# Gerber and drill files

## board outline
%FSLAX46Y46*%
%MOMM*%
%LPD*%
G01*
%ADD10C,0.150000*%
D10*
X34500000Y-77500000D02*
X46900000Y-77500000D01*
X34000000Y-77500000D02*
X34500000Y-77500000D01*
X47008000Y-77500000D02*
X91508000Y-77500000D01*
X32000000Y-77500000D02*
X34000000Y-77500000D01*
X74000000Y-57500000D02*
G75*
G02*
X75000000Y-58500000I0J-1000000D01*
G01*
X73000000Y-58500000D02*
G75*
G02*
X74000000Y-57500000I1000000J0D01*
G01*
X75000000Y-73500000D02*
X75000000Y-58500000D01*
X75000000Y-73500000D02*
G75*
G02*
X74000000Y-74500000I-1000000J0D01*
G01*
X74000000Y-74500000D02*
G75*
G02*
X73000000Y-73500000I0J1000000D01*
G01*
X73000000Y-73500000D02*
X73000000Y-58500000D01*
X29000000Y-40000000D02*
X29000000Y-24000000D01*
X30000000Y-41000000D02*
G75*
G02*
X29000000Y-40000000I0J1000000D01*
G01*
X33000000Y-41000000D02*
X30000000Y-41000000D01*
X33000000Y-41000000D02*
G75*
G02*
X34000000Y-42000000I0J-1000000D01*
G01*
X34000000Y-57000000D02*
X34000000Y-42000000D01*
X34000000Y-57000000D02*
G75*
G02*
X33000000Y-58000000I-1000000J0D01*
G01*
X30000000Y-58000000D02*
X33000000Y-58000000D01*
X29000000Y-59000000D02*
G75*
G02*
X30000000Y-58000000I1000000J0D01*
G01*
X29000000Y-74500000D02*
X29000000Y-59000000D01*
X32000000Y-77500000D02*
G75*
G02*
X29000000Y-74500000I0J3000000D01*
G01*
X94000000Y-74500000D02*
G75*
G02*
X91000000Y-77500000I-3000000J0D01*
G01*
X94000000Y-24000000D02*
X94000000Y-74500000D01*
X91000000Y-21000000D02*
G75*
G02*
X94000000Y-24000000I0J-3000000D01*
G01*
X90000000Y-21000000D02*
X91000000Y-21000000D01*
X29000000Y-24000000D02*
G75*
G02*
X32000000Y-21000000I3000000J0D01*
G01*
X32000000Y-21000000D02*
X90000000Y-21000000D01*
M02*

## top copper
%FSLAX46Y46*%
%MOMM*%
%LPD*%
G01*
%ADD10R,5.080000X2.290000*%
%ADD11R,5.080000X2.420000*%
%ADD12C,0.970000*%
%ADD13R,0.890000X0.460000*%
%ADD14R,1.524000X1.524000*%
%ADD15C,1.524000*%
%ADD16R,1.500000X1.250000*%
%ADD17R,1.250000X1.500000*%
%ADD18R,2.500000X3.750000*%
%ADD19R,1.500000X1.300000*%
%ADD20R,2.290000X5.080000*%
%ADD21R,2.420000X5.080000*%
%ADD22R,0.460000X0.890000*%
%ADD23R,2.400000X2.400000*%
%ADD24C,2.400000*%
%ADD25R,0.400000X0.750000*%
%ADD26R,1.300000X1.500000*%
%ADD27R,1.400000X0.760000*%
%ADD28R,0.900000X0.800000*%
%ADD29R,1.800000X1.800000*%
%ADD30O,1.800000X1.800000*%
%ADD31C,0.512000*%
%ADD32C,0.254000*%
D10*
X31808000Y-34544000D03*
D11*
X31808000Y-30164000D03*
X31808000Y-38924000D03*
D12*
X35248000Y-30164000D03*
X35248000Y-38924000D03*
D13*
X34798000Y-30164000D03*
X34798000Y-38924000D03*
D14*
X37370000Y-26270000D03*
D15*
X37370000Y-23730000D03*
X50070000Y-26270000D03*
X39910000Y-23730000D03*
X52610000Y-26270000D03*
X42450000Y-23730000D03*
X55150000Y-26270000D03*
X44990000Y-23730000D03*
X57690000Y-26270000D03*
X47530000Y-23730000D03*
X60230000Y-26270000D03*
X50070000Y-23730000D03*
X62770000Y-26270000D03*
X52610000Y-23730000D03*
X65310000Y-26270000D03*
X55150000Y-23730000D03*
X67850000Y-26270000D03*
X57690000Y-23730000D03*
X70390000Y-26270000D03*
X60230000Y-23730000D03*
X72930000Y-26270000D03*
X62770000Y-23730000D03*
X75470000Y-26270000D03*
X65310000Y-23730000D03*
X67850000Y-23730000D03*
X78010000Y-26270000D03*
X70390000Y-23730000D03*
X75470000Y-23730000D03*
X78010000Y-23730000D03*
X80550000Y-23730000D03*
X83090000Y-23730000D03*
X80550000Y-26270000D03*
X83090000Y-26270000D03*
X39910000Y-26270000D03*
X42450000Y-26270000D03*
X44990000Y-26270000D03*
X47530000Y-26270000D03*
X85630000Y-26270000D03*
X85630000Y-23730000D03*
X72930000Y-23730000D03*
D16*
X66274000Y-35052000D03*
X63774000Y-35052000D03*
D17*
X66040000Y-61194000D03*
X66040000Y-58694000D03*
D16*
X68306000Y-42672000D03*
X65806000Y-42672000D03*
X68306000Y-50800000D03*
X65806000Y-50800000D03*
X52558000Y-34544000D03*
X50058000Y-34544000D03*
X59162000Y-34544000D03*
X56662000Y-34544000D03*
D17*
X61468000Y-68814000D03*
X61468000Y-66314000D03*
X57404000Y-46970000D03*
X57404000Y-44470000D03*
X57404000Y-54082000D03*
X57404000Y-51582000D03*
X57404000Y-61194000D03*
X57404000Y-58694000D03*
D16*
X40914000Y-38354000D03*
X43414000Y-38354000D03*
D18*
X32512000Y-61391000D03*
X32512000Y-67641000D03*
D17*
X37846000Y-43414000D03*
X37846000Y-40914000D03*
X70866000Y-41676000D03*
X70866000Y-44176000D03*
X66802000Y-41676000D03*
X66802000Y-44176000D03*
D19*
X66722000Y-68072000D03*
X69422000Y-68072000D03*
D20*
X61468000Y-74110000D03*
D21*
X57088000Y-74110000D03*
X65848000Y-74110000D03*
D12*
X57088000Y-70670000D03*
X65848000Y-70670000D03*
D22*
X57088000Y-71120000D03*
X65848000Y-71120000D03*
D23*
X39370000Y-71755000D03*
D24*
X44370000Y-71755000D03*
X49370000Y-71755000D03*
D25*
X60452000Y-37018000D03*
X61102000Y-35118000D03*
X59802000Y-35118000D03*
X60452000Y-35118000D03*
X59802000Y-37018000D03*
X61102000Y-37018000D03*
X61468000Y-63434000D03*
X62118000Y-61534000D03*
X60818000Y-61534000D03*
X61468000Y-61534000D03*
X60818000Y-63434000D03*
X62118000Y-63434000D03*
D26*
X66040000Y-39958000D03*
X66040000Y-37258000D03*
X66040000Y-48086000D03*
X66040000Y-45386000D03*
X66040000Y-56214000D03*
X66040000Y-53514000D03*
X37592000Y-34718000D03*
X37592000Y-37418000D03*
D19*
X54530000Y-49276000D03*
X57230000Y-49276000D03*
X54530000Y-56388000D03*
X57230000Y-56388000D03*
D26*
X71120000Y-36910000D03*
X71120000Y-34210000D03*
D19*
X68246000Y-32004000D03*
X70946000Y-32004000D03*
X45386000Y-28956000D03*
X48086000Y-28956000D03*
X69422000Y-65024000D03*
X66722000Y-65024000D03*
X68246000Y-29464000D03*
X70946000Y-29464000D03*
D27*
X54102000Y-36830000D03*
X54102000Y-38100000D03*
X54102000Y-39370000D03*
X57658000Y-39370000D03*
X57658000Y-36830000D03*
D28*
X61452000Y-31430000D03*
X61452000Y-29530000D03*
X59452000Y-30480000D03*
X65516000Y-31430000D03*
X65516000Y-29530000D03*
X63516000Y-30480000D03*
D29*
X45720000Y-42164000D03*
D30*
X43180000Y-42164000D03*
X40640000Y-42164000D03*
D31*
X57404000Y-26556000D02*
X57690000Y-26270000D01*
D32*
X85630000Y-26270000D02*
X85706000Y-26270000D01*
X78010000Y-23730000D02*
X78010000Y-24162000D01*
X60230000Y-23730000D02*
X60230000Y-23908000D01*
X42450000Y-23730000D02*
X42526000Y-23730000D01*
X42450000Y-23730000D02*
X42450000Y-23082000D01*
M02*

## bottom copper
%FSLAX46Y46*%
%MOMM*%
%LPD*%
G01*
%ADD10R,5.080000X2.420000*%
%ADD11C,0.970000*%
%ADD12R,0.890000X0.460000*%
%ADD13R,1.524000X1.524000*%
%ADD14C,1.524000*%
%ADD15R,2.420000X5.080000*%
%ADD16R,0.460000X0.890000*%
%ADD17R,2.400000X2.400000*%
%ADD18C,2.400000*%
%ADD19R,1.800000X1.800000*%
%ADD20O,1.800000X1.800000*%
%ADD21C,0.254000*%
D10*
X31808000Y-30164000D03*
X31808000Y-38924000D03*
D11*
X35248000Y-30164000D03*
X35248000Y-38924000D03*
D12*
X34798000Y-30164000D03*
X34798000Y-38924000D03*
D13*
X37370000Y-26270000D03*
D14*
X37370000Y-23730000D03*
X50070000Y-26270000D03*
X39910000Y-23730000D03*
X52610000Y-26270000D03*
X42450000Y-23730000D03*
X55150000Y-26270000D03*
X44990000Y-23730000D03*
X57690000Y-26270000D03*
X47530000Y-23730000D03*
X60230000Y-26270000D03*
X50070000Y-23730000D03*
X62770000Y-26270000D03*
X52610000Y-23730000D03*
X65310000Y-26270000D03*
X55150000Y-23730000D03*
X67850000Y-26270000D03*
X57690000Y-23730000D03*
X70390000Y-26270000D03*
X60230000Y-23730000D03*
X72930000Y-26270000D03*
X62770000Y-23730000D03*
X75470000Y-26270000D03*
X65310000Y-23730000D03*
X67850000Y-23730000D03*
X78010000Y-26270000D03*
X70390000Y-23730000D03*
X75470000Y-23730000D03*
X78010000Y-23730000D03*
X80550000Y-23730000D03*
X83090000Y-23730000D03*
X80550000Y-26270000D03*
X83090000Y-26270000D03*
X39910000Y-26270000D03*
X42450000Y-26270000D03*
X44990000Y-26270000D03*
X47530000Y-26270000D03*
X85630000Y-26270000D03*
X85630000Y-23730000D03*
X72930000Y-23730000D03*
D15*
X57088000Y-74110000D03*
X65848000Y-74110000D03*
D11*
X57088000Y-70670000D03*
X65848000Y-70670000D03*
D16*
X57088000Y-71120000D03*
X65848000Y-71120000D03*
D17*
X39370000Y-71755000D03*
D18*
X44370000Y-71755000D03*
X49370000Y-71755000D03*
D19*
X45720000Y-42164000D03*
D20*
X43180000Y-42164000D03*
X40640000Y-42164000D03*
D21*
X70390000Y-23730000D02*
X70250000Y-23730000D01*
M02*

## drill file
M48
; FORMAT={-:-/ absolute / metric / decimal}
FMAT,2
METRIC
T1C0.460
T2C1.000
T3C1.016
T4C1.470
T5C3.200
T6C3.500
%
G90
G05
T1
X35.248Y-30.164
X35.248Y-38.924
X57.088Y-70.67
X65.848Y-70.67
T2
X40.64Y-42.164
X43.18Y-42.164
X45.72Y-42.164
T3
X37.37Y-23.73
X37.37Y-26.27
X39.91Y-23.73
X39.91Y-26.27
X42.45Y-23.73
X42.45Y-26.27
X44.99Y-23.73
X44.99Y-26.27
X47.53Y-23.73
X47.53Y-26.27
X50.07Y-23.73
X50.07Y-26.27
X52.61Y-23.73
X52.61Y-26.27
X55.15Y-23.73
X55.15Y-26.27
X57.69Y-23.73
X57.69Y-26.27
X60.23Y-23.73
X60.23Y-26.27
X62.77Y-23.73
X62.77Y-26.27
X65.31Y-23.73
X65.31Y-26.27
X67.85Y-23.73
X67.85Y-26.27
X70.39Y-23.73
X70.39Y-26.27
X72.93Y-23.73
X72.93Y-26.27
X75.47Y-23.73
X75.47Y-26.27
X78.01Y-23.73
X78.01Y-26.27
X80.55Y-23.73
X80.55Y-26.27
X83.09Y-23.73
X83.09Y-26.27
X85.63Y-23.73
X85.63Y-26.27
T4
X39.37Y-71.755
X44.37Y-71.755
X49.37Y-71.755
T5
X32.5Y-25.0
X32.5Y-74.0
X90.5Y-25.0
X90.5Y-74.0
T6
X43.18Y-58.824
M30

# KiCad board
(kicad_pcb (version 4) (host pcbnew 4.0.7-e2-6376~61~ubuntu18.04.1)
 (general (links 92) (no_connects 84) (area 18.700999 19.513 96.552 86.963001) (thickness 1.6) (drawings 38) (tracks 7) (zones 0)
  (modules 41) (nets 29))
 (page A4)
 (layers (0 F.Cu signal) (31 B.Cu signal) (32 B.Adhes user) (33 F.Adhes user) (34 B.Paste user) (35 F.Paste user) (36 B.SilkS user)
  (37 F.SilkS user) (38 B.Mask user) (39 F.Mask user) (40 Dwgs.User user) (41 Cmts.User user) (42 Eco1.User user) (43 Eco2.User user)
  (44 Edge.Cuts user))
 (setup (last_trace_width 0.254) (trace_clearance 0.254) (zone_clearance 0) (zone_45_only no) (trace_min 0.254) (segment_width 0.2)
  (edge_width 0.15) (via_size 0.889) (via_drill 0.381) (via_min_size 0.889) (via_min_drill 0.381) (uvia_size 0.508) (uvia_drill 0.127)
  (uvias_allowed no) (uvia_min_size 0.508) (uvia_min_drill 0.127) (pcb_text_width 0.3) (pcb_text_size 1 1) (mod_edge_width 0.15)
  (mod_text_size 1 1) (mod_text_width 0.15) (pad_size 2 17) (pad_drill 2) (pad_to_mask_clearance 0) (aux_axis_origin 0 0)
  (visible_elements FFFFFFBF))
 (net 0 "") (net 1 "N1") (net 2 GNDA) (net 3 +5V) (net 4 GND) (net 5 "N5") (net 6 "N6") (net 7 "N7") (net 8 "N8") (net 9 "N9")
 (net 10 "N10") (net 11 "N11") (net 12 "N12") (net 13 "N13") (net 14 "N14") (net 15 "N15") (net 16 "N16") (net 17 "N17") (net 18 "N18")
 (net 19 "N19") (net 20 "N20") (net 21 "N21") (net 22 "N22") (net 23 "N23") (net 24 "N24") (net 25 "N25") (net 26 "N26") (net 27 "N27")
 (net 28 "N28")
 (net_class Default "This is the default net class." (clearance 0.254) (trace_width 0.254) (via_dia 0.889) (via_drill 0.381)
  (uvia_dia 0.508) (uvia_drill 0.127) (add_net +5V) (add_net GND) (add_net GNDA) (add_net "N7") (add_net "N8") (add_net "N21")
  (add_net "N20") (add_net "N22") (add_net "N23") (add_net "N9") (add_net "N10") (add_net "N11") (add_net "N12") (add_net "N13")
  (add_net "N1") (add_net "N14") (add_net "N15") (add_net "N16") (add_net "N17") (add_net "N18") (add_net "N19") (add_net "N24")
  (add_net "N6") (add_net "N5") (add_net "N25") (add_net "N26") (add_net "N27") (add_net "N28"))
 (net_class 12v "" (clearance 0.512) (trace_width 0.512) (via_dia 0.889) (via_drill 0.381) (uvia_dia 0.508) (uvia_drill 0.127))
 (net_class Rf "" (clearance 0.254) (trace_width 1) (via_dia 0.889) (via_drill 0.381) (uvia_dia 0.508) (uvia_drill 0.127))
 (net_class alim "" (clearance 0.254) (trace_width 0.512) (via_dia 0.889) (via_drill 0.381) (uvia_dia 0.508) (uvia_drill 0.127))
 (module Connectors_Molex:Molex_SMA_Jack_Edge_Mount (layer F.Cu) (at 33.528 34.544)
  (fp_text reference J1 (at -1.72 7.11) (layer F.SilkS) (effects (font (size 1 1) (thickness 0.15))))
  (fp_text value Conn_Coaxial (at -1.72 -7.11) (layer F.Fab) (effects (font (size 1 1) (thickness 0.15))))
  (pad 1 smd rect (at -1.72 0) (size 5.08 2.29) (layers F.Cu F.Paste F.Mask) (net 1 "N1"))
  (pad 2 smd rect (at -1.72 -4.38) (size 5.08 2.42) (layers F.Cu F.Paste F.Mask) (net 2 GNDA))
  (pad 2 smd rect (at -1.72 4.38) (size 5.08 2.42) (layers F.Cu F.Paste F.Mask) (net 2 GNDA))
  (pad 2 smd rect (at -1.72 -4.38) (size 5.08 2.42) (layers B.Cu B.Paste B.Mask) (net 2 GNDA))
  (pad 2 smd rect (at -1.72 4.38) (size 5.08 2.42) (layers B.Cu B.Paste B.Mask) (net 2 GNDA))
  (pad 2 thru_hole circle (at 1.72 -4.38) (size 0.97 0.97) (drill 0.46) (layers *.Cu) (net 2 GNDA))
  (pad 2 thru_hole circle (at 1.72 4.38) (size 0.97 0.97) (drill 0.46) (layers *.Cu) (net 2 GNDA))
  (pad 2 smd rect (at 1.27 -4.38) (size 0.89 0.46) (layers F.Cu) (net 2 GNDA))
  (pad 2 smd rect (at 1.27 4.38) (size 0.89 0.46) (layers F.Cu) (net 2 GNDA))
  (pad 2 smd rect (at 1.27 -4.38) (size 0.89 0.46) (layers B.Cu) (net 2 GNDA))
  (pad 2 smd rect (at 1.27 4.38) (size 0.89 0.46) (layers B.Cu) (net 2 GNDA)))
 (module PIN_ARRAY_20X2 (layer F.Cu) (at 61.5 25)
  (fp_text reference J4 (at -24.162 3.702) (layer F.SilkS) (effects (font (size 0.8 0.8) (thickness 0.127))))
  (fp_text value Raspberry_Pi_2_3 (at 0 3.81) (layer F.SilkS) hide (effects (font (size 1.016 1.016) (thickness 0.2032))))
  (pad 1 thru_hole rect (at -24.13 1.27) (size 1.524 1.524) (drill 1.016) (layers *.Cu *.Mask F.SilkS))
  (pad 2 thru_hole circle (at -24.13 -1.27) (size 1.524 1.524) (drill 1.016) (layers *.Cu *.Mask F.SilkS) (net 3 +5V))
  (pad 11 thru_hole circle (at -11.43 1.27) (size 1.524 1.524) (drill 1.016) (layers *.Cu *.Mask F.SilkS))
  (pad 4 thru_hole circle (at -21.59 -1.27) (size 1.524 1.524) (drill 1.016) (layers *.Cu *.Mask F.SilkS) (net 3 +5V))
  (pad 13 thru_hole circle (at -8.89 1.27) (size 1.524 1.524) (drill 1.016) (layers *.Cu *.Mask F.SilkS))
  (pad 6 thru_hole circle (at -19.05 -1.27) (size 1.524 1.524) (drill 1.016) (layers *.Cu *.Mask F.SilkS) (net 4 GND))
  (pad 15 thru_hole circle (at -6.35 1.27) (size 1.524 1.524) (drill 1.016) (layers *.Cu *.Mask F.SilkS))
  (pad 8 thru_hole circle (at -16.51 -1.27) (size 1.524 1.524) (drill 1.016) (layers *.Cu *.Mask F.SilkS) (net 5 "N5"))
  (pad 17 thru_hole circle (at -3.81 1.27) (size 1.524 1.524) (drill 1.016) (layers *.Cu *.Mask F.SilkS))
  (pad 10 thru_hole circle (at -13.97 -1.27) (size 1.524 1.524) (drill 1.016) (layers *.Cu *.Mask F.SilkS) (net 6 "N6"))
  (pad 19 thru_hole circle (at -1.27 1.27) (size 1.524 1.524) (drill 1.016) (layers *.Cu *.Mask F.SilkS))
  (pad 12 thru_hole circle (at -11.43 -1.27) (size 1.524 1.524) (drill 1.016) (layers *.Cu *.Mask F.SilkS))
  (pad 21 thru_hole circle (at 1.27 1.27) (size 1.524 1.524) (drill 1.016) (layers *.Cu *.Mask F.SilkS))
  (pad 14 thru_hole circle (at -8.89 -1.27) (size 1.524 1.524) (drill 1.016) (layers *.Cu *.Mask F.SilkS) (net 4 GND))
  (pad 23 thru_hole circle (at 3.81 1.27) (size 1.524 1.524) (drill 1.016) (layers *.Cu *.Mask F.SilkS))
  (pad 16 thru_hole circle (at -6.35 -1.27) (size 1.524 1.524) (drill 1.016) (layers *.Cu *.Mask F.SilkS))
  (pad 25 thru_hole circle (at 6.35 1.27) (size 1.524 1.524) (drill 1.016) (layers *.Cu *.Mask F.SilkS) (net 4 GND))
  (pad 18 thru_hole circle (at -3.81 -1.27) (size 1.524 1.524) (drill 1.016) (layers *.Cu *.Mask F.SilkS))
  (pad 27 thru_hole circle (at 8.89 1.27) (size 1.524 1.524) (drill 1.016) (layers *.Cu *.Mask F.SilkS))
  (pad 20 thru_hole circle (at -1.27 -1.27) (size 1.524 1.524) (drill 1.016) (layers *.Cu *.Mask F.SilkS) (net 4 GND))
  (pad 29 thru_hole circle (at 11.43 1.27) (size 1.524 1.524) (drill 1.016) (layers *.Cu *.Mask F.SilkS))
  (pad 22 thru_hole circle (at 1.27 -1.27) (size 1.524 1.524) (drill 1.016) (layers *.Cu *.Mask F.SilkS))
  (pad 31 thru_hole circle (at 13.97 1.27) (size 1.524 1.524) (drill 1.016) (layers *.Cu *.Mask F.SilkS))
  (pad 24 thru_hole circle (at 3.81 -1.27) (size 1.524 1.524) (drill 1.016) (layers *.Cu *.Mask F.SilkS))
  (pad 26 thru_hole circle (at 6.35 -1.27) (size 1.524 1.524) (drill 1.016) (layers *.Cu *.Mask F.SilkS))
  (pad 33 thru_hole circle (at 16.51 1.27) (size 1.524 1.524) (drill 1.016) (layers *.Cu *.Mask F.SilkS))
  (pad 28 thru_hole circle (at 8.89 -1.27) (size 1.524 1.524) (drill 1.016) (layers *.Cu *.Mask F.SilkS))
  (pad 32 thru_hole circle (at 13.97 -1.27) (size 1.524 1.524) (drill 1.016) (layers *.Cu *.Mask F.SilkS))
  (pad 34 thru_hole circle (at 16.51 -1.27) (size 1.524 1.524) (drill 1.016) (layers *.Cu *.Mask F.SilkS) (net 4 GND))
  (pad 36 thru_hole circle (at 19.05 -1.27) (size 1.524 1.524) (drill 1.016) (layers *.Cu *.Mask F.SilkS))
  (pad 38 thru_hole circle (at 21.59 -1.27) (size 1.524 1.524) (drill 1.016) (layers *.Cu *.Mask F.SilkS))
  (pad 35 thru_hole circle (at 19.05 1.27) (size 1.524 1.524) (drill 1.016) (layers *.Cu *.Mask F.SilkS))
  (pad 37 thru_hole circle (at 21.59 1.27) (size 1.524 1.524) (drill 1.016) (layers *.Cu *.Mask F.SilkS))
  (pad 3 thru_hole circle (at -21.59 1.27) (size 1.524 1.524) (drill 1.016) (layers *.Cu *.Mask F.SilkS))
  (pad 5 thru_hole circle (at -19.05 1.27) (size 1.524 1.524) (drill 1.016) (layers *.Cu *.Mask F.SilkS))
  (pad 7 thru_hole circle (at -16.51 1.27) (size 1.524 1.524) (drill 1.016) (layers *.Cu *.Mask F.SilkS))
  (pad 9 thru_hole circle (at -13.97 1.27) (size 1.524 1.524) (drill 1.016) (layers *.Cu *.Mask F.SilkS) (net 4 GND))
  (pad 39 thru_hole circle (at 24.13 1.27) (size 1.524 1.524) (drill 1.016) (layers *.Cu *.Mask F.SilkS) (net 4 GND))
  (pad 40 thru_hole circle (at 24.13 -1.27) (size 1.524 1.524) (drill 1.016) (layers *.Cu *.Mask F.SilkS))
  (pad 30 thru_hole circle (at 11.43 -1.27) (size 1.524 1.524) (drill 1.016) (layers *.Cu *.Mask F.SilkS) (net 4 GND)))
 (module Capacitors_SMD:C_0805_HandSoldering (layer F.Cu) (at 65.024 35.052 180)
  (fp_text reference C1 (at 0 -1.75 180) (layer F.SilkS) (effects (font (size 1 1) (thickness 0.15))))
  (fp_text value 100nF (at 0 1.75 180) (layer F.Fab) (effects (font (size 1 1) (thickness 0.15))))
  (pad 1 smd rect (at -1.25 0 180) (size 1.5 1.25) (layers F.Cu F.Paste F.Mask) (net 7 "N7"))
  (pad 2 smd rect (at 1.25 0 180) (size 1.5 1.25) (layers F.Cu F.Paste F.Mask) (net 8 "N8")))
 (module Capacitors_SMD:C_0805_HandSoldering (layer F.Cu) (at 66.04 59.944 90)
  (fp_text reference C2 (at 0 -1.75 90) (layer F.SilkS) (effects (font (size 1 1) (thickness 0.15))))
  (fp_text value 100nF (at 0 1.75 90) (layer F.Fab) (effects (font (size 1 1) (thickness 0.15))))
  (pad 1 smd rect (at -1.25 0 90) (size 1.5 1.25) (layers F.Cu F.Paste F.Mask) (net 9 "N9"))
  (pad 2 smd rect (at 1.25 0 90) (size 1.5 1.25) (layers F.Cu F.Paste F.Mask) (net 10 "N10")))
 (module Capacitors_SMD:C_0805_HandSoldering (layer F.Cu) (at 67.056 42.672 180)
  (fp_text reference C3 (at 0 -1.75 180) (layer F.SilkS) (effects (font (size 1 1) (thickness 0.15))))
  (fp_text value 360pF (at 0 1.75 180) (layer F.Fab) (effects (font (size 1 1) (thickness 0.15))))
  (pad 1 smd rect (at -1.25 0 180) (size 1.5 1.25) (layers F.Cu F.Paste F.Mask) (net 4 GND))
  (pad 2 smd rect (at 1.25 0 180) (size 1.5 1.25) (layers F.Cu F.Paste F.Mask) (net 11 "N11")))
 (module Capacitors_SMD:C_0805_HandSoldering (layer F.Cu) (at 67.056 50.8 180)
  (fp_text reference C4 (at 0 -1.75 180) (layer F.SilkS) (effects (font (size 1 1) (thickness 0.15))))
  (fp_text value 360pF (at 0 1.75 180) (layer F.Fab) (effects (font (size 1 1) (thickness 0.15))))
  (pad 1 smd rect (at -1.25 0 180) (size 1.5 1.25) (layers F.Cu F.Paste F.Mask) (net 4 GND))
  (pad 2 smd rect (at 1.25 0 180) (size 1.5 1.25) (layers F.Cu F.Paste F.Mask) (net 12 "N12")))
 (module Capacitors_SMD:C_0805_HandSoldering (layer F.Cu) (at 51.308 34.544 180)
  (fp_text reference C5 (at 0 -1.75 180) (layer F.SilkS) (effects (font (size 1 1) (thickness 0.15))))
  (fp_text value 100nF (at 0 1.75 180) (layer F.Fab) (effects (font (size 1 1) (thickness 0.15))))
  (pad 1 smd rect (at -1.25 0 180) (size 1.5 1.25) (layers F.Cu F.Paste F.Mask) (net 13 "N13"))
  (pad 2 smd rect (at 1.25 0 180) (size 1.5 1.25) (layers F.Cu F.Paste F.Mask) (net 1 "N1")))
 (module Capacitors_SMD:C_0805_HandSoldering (layer F.Cu) (at 57.912 34.544 180)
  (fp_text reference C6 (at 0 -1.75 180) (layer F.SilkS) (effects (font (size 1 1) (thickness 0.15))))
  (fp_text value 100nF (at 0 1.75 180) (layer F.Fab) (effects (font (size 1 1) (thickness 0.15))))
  (pad 1 smd rect (at -1.25 0 180) (size 1.5 1.25) (layers F.Cu F.Paste F.Mask) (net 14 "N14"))
  (pad 2 smd rect (at 1.25 0 180) (size 1.5 1.25) (layers F.Cu F.Paste F.Mask) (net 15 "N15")))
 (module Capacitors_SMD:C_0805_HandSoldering (layer F.Cu) (at 61.468 67.564 90)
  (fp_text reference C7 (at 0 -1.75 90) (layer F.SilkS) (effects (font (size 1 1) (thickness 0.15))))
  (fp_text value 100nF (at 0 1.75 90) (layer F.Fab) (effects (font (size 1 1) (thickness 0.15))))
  (pad 1 smd rect (at -1.25 0 90) (size 1.5 1.25) (layers F.Cu F.Paste F.Mask) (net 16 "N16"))
  (pad 2 smd rect (at 1.25 0 90) (size 1.5 1.25) (layers F.Cu F.Paste F.Mask) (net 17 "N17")))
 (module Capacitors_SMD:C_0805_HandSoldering (layer F.Cu) (at 57.404 45.72 90)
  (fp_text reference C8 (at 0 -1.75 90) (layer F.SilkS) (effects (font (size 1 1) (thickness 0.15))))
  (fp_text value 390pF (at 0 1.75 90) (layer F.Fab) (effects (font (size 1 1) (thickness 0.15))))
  (pad 1 smd rect (at -1.25 0 90) (size 1.5 1.25) (layers F.Cu F.Paste F.Mask) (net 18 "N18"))
  (pad 2 smd rect (at 1.25 0 90) (size 1.5 1.25) (layers F.Cu F.Paste F.Mask) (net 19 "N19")))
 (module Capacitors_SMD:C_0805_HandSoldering (layer F.Cu) (at 57.404 52.832 90)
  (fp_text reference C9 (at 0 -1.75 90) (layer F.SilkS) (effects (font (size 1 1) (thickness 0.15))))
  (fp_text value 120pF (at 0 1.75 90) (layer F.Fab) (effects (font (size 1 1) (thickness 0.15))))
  (pad 1 smd rect (at -1.25 0 90) (size 1.5 1.25) (layers F.Cu F.Paste F.Mask) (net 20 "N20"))
  (pad 2 smd rect (at 1.25 0 90) (size 1.5 1.25) (layers F.Cu F.Paste F.Mask) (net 18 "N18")))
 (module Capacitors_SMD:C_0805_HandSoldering (layer F.Cu) (at 57.404 59.944 90)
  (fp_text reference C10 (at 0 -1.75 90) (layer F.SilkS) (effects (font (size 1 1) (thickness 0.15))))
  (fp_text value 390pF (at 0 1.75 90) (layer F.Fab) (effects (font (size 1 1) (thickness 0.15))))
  (pad 1 smd rect (at -1.25 0 90) (size 1.5 1.25) (layers F.Cu F.Paste F.Mask) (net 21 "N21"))
  (pad 2 smd rect (at 1.25 0 90) (size 1.5 1.25) (layers F.Cu F.Paste F.Mask) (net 20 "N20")))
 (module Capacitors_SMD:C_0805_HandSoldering (layer F.Cu) (at 42.164 38.354)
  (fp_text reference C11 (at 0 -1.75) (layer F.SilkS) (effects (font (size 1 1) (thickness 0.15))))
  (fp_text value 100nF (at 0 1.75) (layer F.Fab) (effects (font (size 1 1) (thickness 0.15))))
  (pad 1 smd rect (at -1.25 0) (size 1.5 1.25) (layers F.Cu F.Paste F.Mask) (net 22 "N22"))
  (pad 2 smd rect (at 1.25 0) (size 1.5 1.25) (layers F.Cu F.Paste F.Mask) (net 2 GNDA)))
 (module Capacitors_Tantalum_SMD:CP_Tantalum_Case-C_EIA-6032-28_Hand (layer F.Cu) (at 32.512 64.516 270)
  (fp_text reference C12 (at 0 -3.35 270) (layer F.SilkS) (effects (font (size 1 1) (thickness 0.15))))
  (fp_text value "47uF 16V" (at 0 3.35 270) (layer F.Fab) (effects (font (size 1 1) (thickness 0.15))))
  (pad 1 smd rect (at -3.125 0 270) (size 3.75 2.5) (layers F.Cu F.Paste F.Mask) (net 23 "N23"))
  (pad 2 smd rect (at 3.125 0 270) (size 3.75 2.5) (layers F.Cu F.Paste F.Mask) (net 2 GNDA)))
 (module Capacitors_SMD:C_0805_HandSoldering (layer F.Cu) (at 37.846 42.164 90)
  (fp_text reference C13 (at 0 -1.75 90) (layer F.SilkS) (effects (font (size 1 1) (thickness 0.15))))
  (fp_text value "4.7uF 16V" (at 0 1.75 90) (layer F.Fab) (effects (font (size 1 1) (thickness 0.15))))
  (pad 1 smd rect (at -1.25 0 90) (size 1.5 1.25) (layers F.Cu F.Paste F.Mask) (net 22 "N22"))
  (pad 2 smd rect (at 1.25 0 90) (size 1.5 1.25) (layers F.Cu F.Paste F.Mask) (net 2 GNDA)))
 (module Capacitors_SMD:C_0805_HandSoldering (layer F.Cu) (at 70.866 42.926 270)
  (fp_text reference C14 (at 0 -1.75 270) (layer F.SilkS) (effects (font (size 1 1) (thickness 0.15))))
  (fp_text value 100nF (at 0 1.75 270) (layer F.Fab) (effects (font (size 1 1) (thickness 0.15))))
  (pad 1 smd rect (at -1.25 0 270) (size 1.5 1.25) (layers F.Cu F.Paste F.Mask) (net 3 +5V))
  (pad 2 smd rect (at 1.25 0 270) (size 1.5 1.25) (layers F.Cu F.Paste F.Mask) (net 4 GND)))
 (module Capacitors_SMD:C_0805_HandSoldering (layer F.Cu) (at 66.802 42.926 270)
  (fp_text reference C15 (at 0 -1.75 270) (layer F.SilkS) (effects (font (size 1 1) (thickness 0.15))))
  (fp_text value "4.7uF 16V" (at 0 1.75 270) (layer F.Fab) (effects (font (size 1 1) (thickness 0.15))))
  (pad 1 smd rect (at -1.25 0 270) (size 1.5 1.25) (layers F.Cu F.Paste F.Mask) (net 3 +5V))
  (pad 2 smd rect (at 1.25 0 270) (size 1.5 1.25) (layers F.Cu F.Paste F.Mask) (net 4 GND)))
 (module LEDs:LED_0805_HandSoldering (layer F.Cu) (at 68.072 68.072)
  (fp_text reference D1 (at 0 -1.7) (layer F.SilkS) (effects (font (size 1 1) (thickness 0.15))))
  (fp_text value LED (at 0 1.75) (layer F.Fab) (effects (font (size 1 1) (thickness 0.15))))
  (pad 1 smd rect (at -1.35 0) (size 1.5 1.3) (layers F.Cu F.Paste F.Mask) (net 4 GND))
  (pad 2 smd rect (at 1.35 0) (size 1.5 1.3) (layers F.Cu F.Paste F.Mask) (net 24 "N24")))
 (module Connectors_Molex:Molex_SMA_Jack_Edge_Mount (layer F.Cu) (at 61.468 72.39 90)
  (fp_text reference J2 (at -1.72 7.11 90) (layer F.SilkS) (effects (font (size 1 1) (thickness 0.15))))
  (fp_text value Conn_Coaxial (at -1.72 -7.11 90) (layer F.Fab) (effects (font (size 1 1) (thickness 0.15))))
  (pad 1 smd rect (at -1.72 0 90) (size 5.08 2.29) (layers F.Cu F.Paste F.Mask) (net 16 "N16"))
  (pad 2 smd rect (at -1.72 -4.38 90) (size 5.08 2.42) (layers F.Cu F.Paste F.Mask) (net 4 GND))
  (pad 2 smd rect (at -1.72 4.38 90) (size 5.08 2.42) (layers F.Cu F.Paste F.Mask) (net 4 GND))
  (pad 2 smd rect (at -1.72 -4.38 90) (size 5.08 2.42) (layers B.Cu B.Paste B.Mask) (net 4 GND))
  (pad 2 smd rect (at -1.72 4.38 90) (size 5.08 2.42) (layers B.Cu B.Paste B.Mask) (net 4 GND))
  (pad 2 thru_hole circle (at 1.72 -4.38 90) (size 0.97 0.97) (drill 0.46) (layers *.Cu) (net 4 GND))
  (pad 2 thru_hole circle (at 1.72 4.38 90) (size 0.97 0.97) (drill 0.46) (layers *.Cu) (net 4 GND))
  (pad 2 smd rect (at 1.27 -4.38 90) (size 0.89 0.46) (layers F.Cu) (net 4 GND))
  (pad 2 smd rect (at 1.27 4.38 90) (size 0.89 0.46) (layers F.Cu) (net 4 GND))
  (pad 2 smd rect (at 1.27 -4.38 90) (size 0.89 0.46) (layers B.Cu) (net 4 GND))
  (pad 2 smd rect (at 1.27 4.38 90) (size 0.89 0.46) (layers B.Cu) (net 4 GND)))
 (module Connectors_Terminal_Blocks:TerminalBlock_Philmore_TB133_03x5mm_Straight (layer F.Cu) (at 39.37 71.755)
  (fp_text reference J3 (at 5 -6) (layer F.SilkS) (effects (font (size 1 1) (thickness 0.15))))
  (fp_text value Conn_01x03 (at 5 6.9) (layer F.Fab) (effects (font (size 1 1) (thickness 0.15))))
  (pad 1 thru_hole rect (at 0 0) (size 2.4 2.4) (drill 1.47) (layers *.Cu *.Mask) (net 2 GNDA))
  (pad 2 thru_hole circle (at 5 0) (size 2.4 2.4) (drill 1.47) (layers *.Cu *.Mask) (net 23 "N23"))
  (pad 3 thru_hole circle (at 10 0) (size 2.4 2.4) (drill 1.47) (layers *.Cu *.Mask) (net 22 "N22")))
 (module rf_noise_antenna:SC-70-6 (layer F.Cu) (at 60.452 36.068 270)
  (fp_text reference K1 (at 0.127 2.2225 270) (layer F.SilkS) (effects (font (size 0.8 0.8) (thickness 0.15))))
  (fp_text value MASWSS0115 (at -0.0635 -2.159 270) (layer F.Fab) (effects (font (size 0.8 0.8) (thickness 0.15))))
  (pad 5 smd rect (at 0.95 0 90) (size 0.75 0.4) (layers F.Cu F.Paste F.Mask) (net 14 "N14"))
  (pad 1 smd rect (at -0.95 -0.65 90) (size 0.75 0.4) (layers F.Cu F.Paste F.Mask) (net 8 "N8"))
  (pad 3 smd rect (at -0.95 0.65 90) (size 0.75 0.4) (layers F.Cu F.Paste F.Mask) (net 19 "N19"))
  (pad 2 smd rect (at -0.95 0 90) (size 0.75 0.4) (layers F.Cu F.Paste F.Mask) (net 4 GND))
  (pad 4 smd rect (at 0.95 0.65 90) (size 0.75 0.4) (layers F.Cu F.Paste F.Mask) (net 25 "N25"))
  (pad 6 smd rect (at 0.95 -0.65 90) (size 0.75 0.4) (layers F.Cu F.Paste F.Mask) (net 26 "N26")))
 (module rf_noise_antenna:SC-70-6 (layer F.Cu) (at 61.468 62.484 270)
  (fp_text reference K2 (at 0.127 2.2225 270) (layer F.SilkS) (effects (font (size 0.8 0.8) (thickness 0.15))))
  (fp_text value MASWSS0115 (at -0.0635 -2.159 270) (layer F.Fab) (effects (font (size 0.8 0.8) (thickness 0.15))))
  (pad 5 smd rect (at 0.95 0 90) (size 0.75 0.4) (layers F.Cu F.Paste F.Mask) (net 17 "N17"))
  (pad 1 smd rect (at -0.95 -0.65 90) (size 0.75 0.4) (layers F.Cu F.Paste F.Mask) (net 9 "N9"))
  (pad 3 smd rect (at -0.95 0.65 90) (size 0.75 0.4) (layers F.Cu F.Paste F.Mask) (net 21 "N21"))
  (pad 2 smd rect (at -0.95 0 90) (size 0.75 0.4) (layers F.Cu F.Paste F.Mask) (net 4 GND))
  (pad 4 smd rect (at 0.95 0.65 90) (size 0.75 0.4) (layers F.Cu F.Paste F.Mask) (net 25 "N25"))
  (pad 6 smd rect (at 0.95 -0.65 90) (size 0.75 0.4) (layers F.Cu F.Paste F.Mask) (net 26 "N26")))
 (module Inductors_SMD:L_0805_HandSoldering (layer F.Cu) (at 66.04 38.608 90)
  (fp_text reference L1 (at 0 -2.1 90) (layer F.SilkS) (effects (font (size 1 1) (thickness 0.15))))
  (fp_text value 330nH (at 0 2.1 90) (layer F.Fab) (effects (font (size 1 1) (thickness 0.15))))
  (pad 1 smd rect (at -1.35 0 90) (size 1.5 1.3) (layers F.Cu F.Paste F.Mask) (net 11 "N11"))
  (pad 2 smd rect (at 1.35 0 90) (size 1.5 1.3) (layers F.Cu F.Paste F.Mask) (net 7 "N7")))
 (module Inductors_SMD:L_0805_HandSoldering (layer F.Cu) (at 66.04 46.736 90)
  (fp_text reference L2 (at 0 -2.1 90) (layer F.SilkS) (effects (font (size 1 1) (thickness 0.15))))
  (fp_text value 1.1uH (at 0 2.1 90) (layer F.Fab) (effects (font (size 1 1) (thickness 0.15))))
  (pad 1 smd rect (at -1.35 0 90) (size 1.5 1.3) (layers F.Cu F.Paste F.Mask) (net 12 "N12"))
  (pad 2 smd rect (at 1.35 0 90) (size 1.5 1.3) (layers F.Cu F.Paste F.Mask) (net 11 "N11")))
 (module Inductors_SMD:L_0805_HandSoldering (layer F.Cu) (at 66.04 54.864 90)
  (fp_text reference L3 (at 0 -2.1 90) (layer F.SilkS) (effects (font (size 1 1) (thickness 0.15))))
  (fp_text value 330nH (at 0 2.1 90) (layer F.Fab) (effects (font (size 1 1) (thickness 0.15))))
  (pad 1 smd rect (at -1.35 0 90) (size 1.5 1.3) (layers F.Cu F.Paste F.Mask) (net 10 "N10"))
  (pad 2 smd rect (at 1.35 0 90) (size 1.5 1.3) (layers F.Cu F.Paste F.Mask) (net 12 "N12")))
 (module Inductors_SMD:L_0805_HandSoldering (layer F.Cu) (at 37.592 36.068 270)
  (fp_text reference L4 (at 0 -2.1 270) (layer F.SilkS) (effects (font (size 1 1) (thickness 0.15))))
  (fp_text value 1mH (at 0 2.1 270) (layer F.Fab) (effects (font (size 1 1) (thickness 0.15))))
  (pad 1 smd rect (at -1.35 0 270) (size 1.5 1.3) (layers F.Cu F.Paste F.Mask) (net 1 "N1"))
  (pad 2 smd rect (at 1.35 0 270) (size 1.5 1.3) (layers F.Cu F.Paste F.Mask) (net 22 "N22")))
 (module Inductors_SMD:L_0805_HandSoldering (layer F.Cu) (at 55.88 49.276)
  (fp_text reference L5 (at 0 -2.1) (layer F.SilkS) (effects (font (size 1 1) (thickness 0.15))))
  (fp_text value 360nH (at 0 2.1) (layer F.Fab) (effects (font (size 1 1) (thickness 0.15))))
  (pad 1 smd rect (at -1.35 0) (size 1.5 1.3) (layers F.Cu F.Paste F.Mask) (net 4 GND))
  (pad 2 smd rect (at 1.35 0) (size 1.5 1.3) (layers F.Cu F.Paste F.Mask) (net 18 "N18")))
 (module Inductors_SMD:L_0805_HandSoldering (layer F.Cu) (at 55.88 56.388)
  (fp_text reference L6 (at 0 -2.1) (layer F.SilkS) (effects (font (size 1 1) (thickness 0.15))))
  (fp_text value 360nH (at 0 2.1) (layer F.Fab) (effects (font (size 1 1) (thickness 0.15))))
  (pad 1 smd rect (at -1.35 0) (size 1.5 1.3) (layers F.Cu F.Paste F.Mask) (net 4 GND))
  (pad 2 smd rect (at 1.35 0) (size 1.5 1.3) (layers F.Cu F.Paste F.Mask) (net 20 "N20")))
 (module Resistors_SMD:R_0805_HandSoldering (layer F.Cu) (at 71.12 35.56 90)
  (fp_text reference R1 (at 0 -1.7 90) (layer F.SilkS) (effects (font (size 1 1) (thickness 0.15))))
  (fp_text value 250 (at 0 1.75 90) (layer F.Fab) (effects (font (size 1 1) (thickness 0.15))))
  (pad 1 smd rect (at -1.35 0 90) (size 1.5 1.3) (layers F.Cu F.Paste F.Mask) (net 25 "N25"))
  (pad 2 smd rect (at 1.35 0 90) (size 1.5 1.3) (layers F.Cu F.Paste F.Mask) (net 3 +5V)))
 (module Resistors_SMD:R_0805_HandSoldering (layer F.Cu) (at 69.596 32.004)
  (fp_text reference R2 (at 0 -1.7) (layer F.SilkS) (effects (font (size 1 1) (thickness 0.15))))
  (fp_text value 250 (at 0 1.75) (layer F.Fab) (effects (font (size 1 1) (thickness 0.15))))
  (pad 1 smd rect (at -1.35 0) (size 1.5 1.3) (layers F.Cu F.Paste F.Mask) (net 26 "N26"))
  (pad 2 smd rect (at 1.35 0) (size 1.5 1.3) (layers F.Cu F.Paste F.Mask) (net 3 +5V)))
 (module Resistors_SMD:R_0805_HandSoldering (layer F.Cu) (at 46.736 28.956)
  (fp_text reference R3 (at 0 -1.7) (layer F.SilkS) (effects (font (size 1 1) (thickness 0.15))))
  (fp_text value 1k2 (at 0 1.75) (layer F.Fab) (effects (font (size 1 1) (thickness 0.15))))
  (pad 1 smd rect (at -1.35 0) (size 1.5 1.3) (layers F.Cu F.Paste F.Mask) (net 5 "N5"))
  (pad 2 smd rect (at 1.35 0) (size 1.5 1.3) (layers F.Cu F.Paste F.Mask) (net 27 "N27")))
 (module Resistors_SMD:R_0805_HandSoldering (layer F.Cu) (at 68.072 65.024 180)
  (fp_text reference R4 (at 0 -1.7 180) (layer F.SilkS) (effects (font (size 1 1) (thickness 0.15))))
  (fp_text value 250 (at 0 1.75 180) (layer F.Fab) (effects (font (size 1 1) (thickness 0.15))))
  (pad 1 smd rect (at -1.35 0 180) (size 1.5 1.3) (layers F.Cu F.Paste F.Mask) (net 24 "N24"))
  (pad 2 smd rect (at 1.35 0 180) (size 1.5 1.3) (layers F.Cu F.Paste F.Mask) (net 26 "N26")))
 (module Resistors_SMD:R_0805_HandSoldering (layer F.Cu) (at 69.596 29.464)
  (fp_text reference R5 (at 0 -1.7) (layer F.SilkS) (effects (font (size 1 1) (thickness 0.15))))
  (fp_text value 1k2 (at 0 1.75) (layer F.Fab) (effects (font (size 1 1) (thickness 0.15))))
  (pad 1 smd rect (at -1.35 0) (size 1.5 1.3) (layers F.Cu F.Paste F.Mask) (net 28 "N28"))
  (pad 2 smd rect (at 1.35 0) (size 1.5 1.3) (layers F.Cu F.Paste F.Mask) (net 6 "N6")))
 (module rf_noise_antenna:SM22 (layer F.Cu) (at 55.88 38.1)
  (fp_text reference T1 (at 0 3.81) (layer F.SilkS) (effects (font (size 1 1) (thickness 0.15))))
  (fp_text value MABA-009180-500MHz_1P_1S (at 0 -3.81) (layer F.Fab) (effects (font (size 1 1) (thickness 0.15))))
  (pad 1 smd rect (at -1.778 -1.27) (size 1.4 0.76) (layers F.Cu F.Paste F.Mask) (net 13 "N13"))
  (pad 2 smd rect (at -1.778 0) (size 1.4 0.76) (layers F.Cu F.Paste F.Mask))
  (pad 3 smd rect (at -1.778 1.27) (size 1.4 0.76) (layers F.Cu F.Paste F.Mask) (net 2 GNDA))
  (pad 4 smd rect (at 1.778 1.27) (size 1.4 0.76) (layers F.Cu F.Paste F.Mask) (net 4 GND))
  (pad 5 smd rect (at 1.778 -1.27) (size 1.4 0.76) (layers F.Cu F.Paste F.Mask) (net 15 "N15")))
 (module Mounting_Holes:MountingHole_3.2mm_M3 (layer F.Cu) (at 32.5 74)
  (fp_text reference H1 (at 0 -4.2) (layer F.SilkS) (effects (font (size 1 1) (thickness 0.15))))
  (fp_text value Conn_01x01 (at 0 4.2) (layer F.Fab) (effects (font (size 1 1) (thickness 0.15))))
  (pad 1 np_thru_hole circle (at 0 0) (size 3.2 3.2) (drill 3.2) (layers *.Cu *.Mask) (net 4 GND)))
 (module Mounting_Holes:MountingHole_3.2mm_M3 (layer F.Cu) (at 90.5 74)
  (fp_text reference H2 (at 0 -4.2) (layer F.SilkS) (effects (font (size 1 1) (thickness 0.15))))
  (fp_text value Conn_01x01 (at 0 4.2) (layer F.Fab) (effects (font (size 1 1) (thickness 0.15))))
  (pad 1 np_thru_hole circle (at 0 0) (size 3.2 3.2) (drill 3.2) (layers *.Cu *.Mask) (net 4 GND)))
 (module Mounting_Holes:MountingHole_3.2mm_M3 (layer F.Cu) (at 32.5 25)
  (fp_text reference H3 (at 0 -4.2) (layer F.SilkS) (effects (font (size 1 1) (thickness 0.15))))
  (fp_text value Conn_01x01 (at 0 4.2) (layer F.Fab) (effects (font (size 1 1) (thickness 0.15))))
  (pad 1 np_thru_hole circle (at 0 0) (size 3.2 3.2) (drill 3.2) (layers *.Cu *.Mask) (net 4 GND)))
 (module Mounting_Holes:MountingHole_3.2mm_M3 (layer F.Cu) (at 90.5 25)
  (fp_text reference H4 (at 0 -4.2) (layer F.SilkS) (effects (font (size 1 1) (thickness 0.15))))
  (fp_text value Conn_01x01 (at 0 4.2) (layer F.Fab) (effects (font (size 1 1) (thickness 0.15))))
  (pad 1 np_thru_hole circle (at 0 0) (size 3.2 3.2) (drill 3.2) (layers *.Cu *.Mask) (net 4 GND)))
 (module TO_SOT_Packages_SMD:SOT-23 (layer F.Cu) (at 60.452 30.48 180)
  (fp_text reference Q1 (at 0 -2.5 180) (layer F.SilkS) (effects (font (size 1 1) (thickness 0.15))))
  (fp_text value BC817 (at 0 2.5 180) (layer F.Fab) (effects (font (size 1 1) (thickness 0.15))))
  (pad 1 smd rect (at -1 -0.95 180) (size 0.9 0.8) (layers F.Cu F.Paste F.Mask) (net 4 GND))
  (pad 2 smd rect (at -1 0.95 180) (size 0.9 0.8) (layers F.Cu F.Paste F.Mask) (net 27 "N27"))
  (pad 3 smd rect (at 1 0 180) (size 0.9 0.8) (layers F.Cu F.Paste F.Mask) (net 25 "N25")))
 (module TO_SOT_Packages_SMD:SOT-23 (layer F.Cu) (at 64.516 30.48 180)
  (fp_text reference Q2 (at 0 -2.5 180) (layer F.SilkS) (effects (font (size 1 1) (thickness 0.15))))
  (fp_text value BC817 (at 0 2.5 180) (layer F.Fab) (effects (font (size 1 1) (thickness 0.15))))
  (pad 1 smd rect (at -1 -0.95 180) (size 0.9 0.8) (layers F.Cu F.Paste F.Mask) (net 4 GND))
  (pad 2 smd rect (at -1 0.95 180) (size 0.9 0.8) (layers F.Cu F.Paste F.Mask) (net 28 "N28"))
  (pad 3 smd rect (at 1 0 180) (size 0.9 0.8) (layers F.Cu F.Paste F.Mask) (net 26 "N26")))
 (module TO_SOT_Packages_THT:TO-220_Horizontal (layer F.Cu) (at 45.72 42.164 180)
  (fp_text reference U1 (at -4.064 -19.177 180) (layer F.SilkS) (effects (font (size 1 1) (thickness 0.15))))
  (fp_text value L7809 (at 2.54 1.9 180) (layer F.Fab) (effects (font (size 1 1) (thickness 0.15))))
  (pad 0 np_thru_hole oval (at 2.54 -16.66 180) (size 3.5 3.5) (drill 3.5) (layers *.Cu *.Mask))
  (pad 1 thru_hole rect (at 0 0 180) (size 1.8 1.8) (drill 1) (layers *.Cu *.Mask) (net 23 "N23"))
  (pad 2 thru_hole oval (at 2.54 0 180) (size 1.8 1.8) (drill 1) (layers *.Cu *.Mask) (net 2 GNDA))
  (pad 3 thru_hole oval (at 5.08 0 180) (size 1.8 1.8) (drill 1) (layers *.Cu *.Mask) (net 22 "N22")))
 (gr_line (start 34.5 77.5) (end 46.9 77.5) (angle 90) (layer Edge.Cuts) (width 0.15))
 (gr_line (start 34 77.5) (end 34.5 77.5) (angle 90) (layer Edge.Cuts) (width 0.15))
 (gr_line (start 47.008 77.5) (end 91.508 77.5) (angle 90) (layer Edge.Cuts) (width 0.15))
 (gr_line (start 32 77.5) (end 34 77.5) (angle 90) (layer Edge.Cuts) (width 0.15))
 (gr_arc (start 74 58.5) (end 74 57.5) (angle 90) (layer Edge.Cuts) (width 0.15))
 (gr_arc (start 74 58.5) (end 73 58.5) (angle 90) (layer Edge.Cuts) (width 0.15))
 (gr_line (start 75 73.5) (end 75 58.5) (angle 90) (layer Edge.Cuts) (width 0.15))
 (gr_arc (start 74 73.5) (end 75 73.5) (angle 90) (layer Edge.Cuts) (width 0.15))
 (gr_arc (start 74 73.5) (end 74 74.5) (angle 90) (layer Edge.Cuts) (width 0.15))
 (gr_line (start 73 73.5) (end 73 58.5) (angle 90) (layer Edge.Cuts) (width 0.15))
 (gr_line (start 29 40) (end 29 24) (angle 90) (layer Edge.Cuts) (width 0.15))
 (gr_arc (start 30 40) (end 30 41) (angle 90) (layer Edge.Cuts) (width 0.15))
 (gr_line (start 33 41) (end 30 41) (angle 90) (layer Edge.Cuts) (width 0.15))
 (gr_arc (start 33 42) (end 33 41) (angle 90) (layer Edge.Cuts) (width 0.15))
 (gr_line (start 34 57) (end 34 42) (angle 90) (layer Edge.Cuts) (width 0.15))
 (gr_arc (start 33 57) (end 34 57) (angle 90) (layer Edge.Cuts) (width 0.15))
 (gr_line (start 30 58) (end 33 58) (angle 90) (layer Edge.Cuts) (width 0.15))
 (gr_arc (start 30 59) (end 29 59) (angle 90) (layer Edge.Cuts) (width 0.15))
 (gr_line (start 29 74.5) (end 29 59) (angle 90) (layer Edge.Cuts) (width 0.15))
 (gr_arc (start 32 74.5) (end 32 77.5) (angle 90) (layer Edge.Cuts) (width 0.15))
 (gr_arc (start 91 74.5) (end 94 74.5) (angle 90) (layer Edge.Cuts) (width 0.15))
 (gr_line (start 94 24) (end 94 74.5) (angle 90) (layer Edge.Cuts) (width 0.15))
 (gr_arc (start 91 24) (end 91 21) (angle 90) (layer Edge.Cuts) (width 0.15))
 (gr_line (start 90 21) (end 91 21) (angle 90) (layer Edge.Cuts) (width 0.15))
 (gr_arc (start 32 24) (end 29 24) (angle 90) (layer Edge.Cuts) (width 0.15))
 (gr_line (start 32 21) (end 90 21) (angle 90) (layer Edge.Cuts) (width 0.15))
 (segment (start 57.404 26.556) (end 57.69 26.27) (width 0.512) (layer F.Cu) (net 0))
 (segment (start 70.39 23.73) (end 70.25 23.73) (width 0.254) (layer B.Cu) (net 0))
 (segment (start 85.63 26.27) (end 85.706 26.27) (width 0.254) (layer F.Cu) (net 4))
 (segment (start 78.01 23.73) (end 78.01 24.162) (width 0.254) (layer F.Cu) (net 4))
 (segment (start 60.23 23.73) (end 60.23 23.908) (width 0.254) (layer F.Cu) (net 4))
 (segment (start 42.45 23.73) (end 42.526 23.73) (width 0.254) (layer F.Cu) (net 4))
 (segment (start 42.45 23.73) (end 42.45 23.082) (width 0.254) (layer F.Cu) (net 4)))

